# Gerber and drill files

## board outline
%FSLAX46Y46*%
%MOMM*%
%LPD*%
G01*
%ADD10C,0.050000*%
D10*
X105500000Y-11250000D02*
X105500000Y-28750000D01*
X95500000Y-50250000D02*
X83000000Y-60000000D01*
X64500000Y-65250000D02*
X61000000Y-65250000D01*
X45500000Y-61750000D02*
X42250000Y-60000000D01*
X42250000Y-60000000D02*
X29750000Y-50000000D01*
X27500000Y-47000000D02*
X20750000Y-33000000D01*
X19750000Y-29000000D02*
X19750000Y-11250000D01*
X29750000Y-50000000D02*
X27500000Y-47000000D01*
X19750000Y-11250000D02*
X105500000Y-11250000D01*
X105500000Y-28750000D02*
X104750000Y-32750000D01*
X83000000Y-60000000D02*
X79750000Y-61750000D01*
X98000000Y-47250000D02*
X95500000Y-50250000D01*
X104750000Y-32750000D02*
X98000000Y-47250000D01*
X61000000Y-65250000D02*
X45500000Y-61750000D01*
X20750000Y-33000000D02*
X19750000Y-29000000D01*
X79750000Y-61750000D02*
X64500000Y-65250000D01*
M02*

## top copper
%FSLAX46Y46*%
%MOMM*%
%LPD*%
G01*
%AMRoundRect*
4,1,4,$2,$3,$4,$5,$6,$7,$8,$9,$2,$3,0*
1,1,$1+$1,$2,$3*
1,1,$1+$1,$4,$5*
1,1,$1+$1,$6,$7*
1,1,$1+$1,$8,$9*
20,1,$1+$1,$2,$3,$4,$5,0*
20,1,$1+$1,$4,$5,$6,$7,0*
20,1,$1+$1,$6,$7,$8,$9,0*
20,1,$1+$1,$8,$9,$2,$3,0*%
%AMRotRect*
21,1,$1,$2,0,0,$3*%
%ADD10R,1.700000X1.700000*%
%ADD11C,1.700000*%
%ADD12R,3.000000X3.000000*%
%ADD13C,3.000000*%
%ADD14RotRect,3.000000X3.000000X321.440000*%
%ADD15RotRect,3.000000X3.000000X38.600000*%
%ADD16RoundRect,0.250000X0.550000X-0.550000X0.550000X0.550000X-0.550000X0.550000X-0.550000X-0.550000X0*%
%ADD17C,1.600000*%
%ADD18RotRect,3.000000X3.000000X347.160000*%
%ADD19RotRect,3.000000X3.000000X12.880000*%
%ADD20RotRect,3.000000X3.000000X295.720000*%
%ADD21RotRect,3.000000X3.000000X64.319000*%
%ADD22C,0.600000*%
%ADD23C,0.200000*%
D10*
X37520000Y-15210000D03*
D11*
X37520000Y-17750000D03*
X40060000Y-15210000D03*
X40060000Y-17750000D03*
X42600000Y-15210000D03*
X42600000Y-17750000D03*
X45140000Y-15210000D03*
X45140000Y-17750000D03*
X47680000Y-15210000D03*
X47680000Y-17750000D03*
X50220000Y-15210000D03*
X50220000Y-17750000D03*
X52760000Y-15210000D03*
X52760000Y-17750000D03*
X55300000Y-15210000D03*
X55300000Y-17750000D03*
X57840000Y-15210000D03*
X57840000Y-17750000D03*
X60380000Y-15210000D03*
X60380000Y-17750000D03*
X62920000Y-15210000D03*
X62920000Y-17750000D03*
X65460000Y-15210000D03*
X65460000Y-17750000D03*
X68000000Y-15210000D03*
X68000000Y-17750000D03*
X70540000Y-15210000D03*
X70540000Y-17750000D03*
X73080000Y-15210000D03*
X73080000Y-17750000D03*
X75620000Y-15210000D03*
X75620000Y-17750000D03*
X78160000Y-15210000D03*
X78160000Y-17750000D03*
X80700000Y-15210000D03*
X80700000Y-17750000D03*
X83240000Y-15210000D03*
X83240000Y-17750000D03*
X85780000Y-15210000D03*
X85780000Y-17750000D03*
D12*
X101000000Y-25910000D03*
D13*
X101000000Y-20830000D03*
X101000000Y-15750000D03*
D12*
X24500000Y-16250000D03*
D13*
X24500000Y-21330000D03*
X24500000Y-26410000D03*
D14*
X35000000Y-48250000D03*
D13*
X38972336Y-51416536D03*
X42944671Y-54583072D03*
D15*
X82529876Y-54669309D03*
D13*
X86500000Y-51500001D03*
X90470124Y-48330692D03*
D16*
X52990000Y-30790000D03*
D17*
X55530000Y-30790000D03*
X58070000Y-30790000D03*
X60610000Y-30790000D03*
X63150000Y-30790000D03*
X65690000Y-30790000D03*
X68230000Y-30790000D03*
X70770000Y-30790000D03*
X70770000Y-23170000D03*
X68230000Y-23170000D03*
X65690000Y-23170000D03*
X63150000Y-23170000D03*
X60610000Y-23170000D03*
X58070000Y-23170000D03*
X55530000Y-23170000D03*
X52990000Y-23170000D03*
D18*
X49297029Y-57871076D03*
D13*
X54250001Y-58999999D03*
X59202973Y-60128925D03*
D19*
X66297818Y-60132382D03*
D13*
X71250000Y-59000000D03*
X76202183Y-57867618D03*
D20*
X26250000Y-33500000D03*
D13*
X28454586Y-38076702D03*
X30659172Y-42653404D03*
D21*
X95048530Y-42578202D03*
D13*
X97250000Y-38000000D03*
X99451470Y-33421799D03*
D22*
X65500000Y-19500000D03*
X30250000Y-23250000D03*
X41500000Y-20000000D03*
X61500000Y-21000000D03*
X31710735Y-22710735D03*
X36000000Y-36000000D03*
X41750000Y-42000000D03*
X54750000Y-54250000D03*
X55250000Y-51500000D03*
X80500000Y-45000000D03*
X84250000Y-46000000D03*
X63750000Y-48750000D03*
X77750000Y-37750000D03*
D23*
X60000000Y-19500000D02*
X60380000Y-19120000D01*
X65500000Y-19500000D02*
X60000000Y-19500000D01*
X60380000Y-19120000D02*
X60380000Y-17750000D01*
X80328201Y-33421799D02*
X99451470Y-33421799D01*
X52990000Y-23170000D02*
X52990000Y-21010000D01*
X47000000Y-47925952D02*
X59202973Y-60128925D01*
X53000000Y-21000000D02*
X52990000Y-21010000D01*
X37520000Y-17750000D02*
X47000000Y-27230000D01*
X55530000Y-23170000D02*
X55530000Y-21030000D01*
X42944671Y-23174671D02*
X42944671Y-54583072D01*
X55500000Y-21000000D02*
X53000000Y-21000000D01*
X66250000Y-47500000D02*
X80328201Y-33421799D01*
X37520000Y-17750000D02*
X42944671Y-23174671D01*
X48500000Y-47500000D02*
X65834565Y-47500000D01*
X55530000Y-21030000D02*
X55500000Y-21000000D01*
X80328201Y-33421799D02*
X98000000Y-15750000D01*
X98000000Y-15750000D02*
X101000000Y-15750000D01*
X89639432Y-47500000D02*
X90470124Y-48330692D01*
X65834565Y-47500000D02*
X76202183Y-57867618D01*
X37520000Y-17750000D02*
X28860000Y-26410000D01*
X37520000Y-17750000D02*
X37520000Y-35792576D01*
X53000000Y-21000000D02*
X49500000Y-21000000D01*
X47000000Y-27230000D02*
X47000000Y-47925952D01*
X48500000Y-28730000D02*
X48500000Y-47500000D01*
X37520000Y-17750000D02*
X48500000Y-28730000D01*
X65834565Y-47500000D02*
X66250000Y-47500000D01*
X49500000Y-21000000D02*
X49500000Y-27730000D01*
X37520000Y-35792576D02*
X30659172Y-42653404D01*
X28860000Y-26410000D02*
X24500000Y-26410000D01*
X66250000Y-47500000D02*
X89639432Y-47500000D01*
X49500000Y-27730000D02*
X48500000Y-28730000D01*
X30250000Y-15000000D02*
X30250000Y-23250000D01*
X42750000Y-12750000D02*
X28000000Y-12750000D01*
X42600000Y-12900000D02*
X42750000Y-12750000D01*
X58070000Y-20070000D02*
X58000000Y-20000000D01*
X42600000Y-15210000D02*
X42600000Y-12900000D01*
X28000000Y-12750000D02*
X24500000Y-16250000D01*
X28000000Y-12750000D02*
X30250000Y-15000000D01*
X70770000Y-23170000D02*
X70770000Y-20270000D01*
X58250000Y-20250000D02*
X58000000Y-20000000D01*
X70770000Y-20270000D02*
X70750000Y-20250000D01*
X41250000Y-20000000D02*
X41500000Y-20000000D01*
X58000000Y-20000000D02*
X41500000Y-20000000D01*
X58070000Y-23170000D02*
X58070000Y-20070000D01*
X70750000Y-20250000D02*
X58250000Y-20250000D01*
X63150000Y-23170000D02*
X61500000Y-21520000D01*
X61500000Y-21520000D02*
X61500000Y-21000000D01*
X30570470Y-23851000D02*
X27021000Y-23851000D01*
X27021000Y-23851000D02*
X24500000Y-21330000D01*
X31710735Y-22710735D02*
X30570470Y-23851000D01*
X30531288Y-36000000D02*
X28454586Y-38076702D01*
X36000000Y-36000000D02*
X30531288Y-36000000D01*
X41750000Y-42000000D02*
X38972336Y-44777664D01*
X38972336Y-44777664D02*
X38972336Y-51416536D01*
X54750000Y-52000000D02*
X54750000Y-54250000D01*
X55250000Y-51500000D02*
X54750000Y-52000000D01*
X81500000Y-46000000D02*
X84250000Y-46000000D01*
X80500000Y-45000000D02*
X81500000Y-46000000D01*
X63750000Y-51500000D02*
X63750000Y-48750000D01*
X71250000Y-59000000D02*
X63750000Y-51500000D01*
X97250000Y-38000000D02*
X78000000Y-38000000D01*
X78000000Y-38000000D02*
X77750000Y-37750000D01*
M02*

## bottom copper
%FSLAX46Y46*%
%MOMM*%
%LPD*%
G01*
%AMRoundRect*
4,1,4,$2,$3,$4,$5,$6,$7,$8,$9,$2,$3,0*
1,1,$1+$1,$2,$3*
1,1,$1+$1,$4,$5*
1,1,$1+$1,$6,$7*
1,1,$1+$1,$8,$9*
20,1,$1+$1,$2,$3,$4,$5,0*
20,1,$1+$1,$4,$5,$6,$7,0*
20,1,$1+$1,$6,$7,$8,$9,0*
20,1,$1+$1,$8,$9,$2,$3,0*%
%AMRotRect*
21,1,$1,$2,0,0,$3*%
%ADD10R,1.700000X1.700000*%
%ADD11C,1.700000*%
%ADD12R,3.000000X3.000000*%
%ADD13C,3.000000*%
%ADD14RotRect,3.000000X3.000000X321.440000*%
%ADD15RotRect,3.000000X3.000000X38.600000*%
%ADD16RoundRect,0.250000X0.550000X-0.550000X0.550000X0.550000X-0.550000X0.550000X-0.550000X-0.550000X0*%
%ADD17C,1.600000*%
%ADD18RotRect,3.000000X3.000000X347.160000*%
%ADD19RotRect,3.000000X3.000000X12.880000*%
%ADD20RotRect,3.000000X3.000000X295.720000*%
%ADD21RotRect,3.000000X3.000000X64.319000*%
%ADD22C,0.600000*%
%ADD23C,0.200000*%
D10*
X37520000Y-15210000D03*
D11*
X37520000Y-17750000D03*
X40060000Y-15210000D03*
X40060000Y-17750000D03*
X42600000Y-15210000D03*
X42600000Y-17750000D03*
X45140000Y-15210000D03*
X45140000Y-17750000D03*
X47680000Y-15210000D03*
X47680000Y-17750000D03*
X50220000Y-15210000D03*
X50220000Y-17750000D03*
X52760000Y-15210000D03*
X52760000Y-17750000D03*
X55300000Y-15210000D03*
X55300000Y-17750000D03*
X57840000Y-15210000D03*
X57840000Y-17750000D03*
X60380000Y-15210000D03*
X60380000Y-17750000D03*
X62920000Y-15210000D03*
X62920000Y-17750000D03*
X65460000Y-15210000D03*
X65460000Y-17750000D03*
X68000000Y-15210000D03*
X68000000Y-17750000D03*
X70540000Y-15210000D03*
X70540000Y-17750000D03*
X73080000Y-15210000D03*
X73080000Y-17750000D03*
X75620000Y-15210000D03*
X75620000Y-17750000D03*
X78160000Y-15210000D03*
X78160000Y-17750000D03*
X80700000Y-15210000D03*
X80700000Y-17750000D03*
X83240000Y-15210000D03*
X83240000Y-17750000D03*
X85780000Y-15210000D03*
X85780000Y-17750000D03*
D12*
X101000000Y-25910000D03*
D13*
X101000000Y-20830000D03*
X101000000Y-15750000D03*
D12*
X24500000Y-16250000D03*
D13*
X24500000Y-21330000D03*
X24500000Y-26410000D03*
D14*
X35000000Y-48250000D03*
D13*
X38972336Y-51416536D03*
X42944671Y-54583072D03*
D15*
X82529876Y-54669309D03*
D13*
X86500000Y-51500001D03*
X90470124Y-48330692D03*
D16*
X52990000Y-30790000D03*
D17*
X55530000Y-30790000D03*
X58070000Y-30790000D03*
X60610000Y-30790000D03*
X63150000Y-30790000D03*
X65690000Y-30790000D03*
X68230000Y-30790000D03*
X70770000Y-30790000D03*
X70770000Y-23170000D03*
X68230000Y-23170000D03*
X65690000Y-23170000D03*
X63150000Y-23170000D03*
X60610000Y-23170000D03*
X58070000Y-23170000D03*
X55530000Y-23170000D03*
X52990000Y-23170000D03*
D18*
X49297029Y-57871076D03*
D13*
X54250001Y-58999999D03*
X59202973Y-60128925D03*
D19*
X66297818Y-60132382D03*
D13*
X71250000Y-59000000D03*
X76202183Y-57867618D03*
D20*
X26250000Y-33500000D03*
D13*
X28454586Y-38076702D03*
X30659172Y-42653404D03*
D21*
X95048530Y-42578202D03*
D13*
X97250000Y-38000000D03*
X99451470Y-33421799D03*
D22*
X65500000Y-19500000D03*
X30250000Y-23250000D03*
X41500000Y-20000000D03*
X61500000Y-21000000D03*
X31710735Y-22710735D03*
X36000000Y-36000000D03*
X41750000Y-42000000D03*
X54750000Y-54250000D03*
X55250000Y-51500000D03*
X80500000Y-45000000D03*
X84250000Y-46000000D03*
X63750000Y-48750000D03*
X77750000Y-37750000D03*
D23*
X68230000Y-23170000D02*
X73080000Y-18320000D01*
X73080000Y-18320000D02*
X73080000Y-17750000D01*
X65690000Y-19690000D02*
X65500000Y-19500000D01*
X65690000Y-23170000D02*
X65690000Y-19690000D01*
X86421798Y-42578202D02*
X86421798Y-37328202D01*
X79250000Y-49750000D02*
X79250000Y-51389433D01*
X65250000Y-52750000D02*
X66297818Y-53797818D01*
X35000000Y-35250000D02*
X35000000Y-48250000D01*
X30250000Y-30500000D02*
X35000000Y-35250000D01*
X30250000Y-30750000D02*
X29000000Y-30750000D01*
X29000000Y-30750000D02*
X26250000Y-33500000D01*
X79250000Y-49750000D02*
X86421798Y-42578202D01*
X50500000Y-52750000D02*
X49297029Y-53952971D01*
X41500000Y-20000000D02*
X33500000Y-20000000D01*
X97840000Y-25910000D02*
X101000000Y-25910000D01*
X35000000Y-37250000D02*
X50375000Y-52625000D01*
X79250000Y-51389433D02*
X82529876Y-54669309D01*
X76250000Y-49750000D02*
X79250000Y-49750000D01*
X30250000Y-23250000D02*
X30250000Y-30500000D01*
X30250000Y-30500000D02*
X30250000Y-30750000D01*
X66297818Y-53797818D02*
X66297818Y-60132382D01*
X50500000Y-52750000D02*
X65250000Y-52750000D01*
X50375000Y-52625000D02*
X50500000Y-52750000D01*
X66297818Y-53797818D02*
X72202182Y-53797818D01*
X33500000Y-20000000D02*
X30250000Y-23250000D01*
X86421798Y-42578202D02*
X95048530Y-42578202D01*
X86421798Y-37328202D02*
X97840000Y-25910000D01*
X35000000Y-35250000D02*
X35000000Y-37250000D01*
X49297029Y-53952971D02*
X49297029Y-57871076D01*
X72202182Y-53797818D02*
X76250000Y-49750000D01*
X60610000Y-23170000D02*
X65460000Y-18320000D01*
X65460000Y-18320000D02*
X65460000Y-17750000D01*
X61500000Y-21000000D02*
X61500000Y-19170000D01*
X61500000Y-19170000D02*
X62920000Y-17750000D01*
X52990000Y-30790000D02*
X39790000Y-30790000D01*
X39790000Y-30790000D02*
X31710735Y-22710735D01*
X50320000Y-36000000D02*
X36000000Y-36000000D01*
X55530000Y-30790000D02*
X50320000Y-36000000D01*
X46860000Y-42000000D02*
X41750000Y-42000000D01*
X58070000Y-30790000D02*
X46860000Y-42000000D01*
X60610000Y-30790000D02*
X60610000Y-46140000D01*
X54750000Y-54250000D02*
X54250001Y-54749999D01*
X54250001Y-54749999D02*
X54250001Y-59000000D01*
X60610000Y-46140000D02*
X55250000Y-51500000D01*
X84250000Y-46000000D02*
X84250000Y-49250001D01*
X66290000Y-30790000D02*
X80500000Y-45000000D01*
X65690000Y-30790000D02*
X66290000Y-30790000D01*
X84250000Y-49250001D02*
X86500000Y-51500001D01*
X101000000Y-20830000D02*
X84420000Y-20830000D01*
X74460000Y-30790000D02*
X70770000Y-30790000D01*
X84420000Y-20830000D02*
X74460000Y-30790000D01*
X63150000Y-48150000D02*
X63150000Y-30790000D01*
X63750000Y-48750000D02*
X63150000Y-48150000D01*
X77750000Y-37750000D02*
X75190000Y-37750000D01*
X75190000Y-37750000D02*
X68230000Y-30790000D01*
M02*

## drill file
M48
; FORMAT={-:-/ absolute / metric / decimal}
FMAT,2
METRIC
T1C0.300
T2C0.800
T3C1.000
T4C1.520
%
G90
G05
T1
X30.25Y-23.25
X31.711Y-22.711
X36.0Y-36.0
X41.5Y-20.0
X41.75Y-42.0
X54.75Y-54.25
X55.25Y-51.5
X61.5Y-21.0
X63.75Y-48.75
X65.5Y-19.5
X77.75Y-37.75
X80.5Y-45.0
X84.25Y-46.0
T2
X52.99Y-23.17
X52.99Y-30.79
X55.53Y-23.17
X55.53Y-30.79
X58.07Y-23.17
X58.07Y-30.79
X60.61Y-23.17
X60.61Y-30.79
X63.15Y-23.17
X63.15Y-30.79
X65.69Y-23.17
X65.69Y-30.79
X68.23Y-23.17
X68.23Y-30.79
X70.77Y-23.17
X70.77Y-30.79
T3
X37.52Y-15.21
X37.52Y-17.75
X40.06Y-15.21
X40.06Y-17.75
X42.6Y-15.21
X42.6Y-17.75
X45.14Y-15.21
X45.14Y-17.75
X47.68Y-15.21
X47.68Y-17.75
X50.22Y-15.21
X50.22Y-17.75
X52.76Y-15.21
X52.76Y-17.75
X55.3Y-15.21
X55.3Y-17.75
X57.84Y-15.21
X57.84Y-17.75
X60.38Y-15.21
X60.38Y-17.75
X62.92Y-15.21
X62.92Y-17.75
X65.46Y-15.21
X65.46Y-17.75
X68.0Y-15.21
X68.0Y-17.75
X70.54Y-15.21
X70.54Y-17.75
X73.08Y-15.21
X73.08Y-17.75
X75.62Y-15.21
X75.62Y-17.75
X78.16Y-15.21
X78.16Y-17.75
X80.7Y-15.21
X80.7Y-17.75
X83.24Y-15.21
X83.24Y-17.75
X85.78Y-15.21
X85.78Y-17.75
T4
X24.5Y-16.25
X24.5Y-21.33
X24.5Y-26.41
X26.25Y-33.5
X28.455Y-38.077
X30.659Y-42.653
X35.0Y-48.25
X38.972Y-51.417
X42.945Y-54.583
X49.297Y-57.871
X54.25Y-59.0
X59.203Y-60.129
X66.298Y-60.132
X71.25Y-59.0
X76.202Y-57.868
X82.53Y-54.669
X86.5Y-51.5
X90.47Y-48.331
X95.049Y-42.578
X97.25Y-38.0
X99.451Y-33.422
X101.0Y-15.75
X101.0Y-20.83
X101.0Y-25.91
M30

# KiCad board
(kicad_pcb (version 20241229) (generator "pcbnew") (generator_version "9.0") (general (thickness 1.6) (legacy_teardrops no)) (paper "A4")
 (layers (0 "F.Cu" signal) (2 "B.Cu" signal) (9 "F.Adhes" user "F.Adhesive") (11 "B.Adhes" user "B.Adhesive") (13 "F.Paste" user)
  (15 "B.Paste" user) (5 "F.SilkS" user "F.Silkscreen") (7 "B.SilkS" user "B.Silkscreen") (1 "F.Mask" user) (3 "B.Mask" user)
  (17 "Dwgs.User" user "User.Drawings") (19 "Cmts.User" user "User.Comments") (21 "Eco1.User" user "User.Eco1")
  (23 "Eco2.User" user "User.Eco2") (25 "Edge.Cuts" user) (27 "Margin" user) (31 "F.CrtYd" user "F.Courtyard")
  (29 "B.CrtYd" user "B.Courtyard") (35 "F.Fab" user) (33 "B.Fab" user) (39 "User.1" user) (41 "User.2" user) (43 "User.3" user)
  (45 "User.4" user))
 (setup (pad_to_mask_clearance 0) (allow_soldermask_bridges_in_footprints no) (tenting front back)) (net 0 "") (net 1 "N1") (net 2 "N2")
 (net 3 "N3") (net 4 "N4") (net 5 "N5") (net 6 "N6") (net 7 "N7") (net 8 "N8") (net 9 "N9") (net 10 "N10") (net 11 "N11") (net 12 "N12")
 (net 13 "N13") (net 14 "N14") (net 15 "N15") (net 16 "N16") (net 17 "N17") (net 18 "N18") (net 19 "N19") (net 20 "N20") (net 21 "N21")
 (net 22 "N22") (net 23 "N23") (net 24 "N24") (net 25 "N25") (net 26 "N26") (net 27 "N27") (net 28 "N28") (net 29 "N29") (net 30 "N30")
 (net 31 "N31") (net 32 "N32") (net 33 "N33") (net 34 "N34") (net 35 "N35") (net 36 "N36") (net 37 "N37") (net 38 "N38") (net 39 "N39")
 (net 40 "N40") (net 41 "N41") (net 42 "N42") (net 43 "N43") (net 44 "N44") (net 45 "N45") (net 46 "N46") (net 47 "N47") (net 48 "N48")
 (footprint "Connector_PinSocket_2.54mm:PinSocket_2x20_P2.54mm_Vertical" (layer "F.Cu") (at 37.52 15.21 90)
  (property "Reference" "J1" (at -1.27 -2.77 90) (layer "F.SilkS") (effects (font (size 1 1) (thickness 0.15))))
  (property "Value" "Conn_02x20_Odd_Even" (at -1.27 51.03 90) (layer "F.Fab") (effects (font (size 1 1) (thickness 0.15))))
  (pad "1" thru_hole rect (at 0 0 90) (size 1.7 1.7) (drill 1) (layers "*.Cu" "*.Mask") (remove_unused_layers no) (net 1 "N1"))
  (pad "2" thru_hole circle (at -2.54 0 90) (size 1.7 1.7) (drill 1) (layers "*.Cu" "*.Mask") (remove_unused_layers no) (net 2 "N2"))
  (pad "3" thru_hole circle (at 0 2.54 90) (size 1.7 1.7) (drill 1) (layers "*.Cu" "*.Mask") (remove_unused_layers no) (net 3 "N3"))
  (pad "4" thru_hole circle (at -2.54 2.54 90) (size 1.7 1.7) (drill 1) (layers "*.Cu" "*.Mask") (remove_unused_layers no) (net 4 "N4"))
  (pad "5" thru_hole circle (at 0 5.08 90) (size 1.7 1.7) (drill 1) (layers "*.Cu" "*.Mask") (remove_unused_layers no) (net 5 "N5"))
  (pad "6" thru_hole circle (at -2.54 5.08 90) (size 1.7 1.7) (drill 1) (layers "*.Cu" "*.Mask") (remove_unused_layers no) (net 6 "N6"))
  (pad "7" thru_hole circle (at 0 7.62 90) (size 1.7 1.7) (drill 1) (layers "*.Cu" "*.Mask") (remove_unused_layers no) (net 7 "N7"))
  (pad "8" thru_hole circle (at -2.54 7.62 90) (size 1.7 1.7) (drill 1) (layers "*.Cu" "*.Mask") (remove_unused_layers no) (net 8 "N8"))
  (pad "9" thru_hole circle (at 0 10.16 90) (size 1.7 1.7) (drill 1) (layers "*.Cu" "*.Mask") (remove_unused_layers no) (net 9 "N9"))
  (pad "10" thru_hole circle (at -2.54 10.16 90) (size 1.7 1.7) (drill 1) (layers "*.Cu" "*.Mask") (remove_unused_layers no) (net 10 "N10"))
  (pad "11" thru_hole circle (at 0 12.7 90) (size 1.7 1.7) (drill 1) (layers "*.Cu" "*.Mask") (remove_unused_layers no) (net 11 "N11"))
  (pad "12" thru_hole circle (at -2.54 12.7 90) (size 1.7 1.7) (drill 1) (layers "*.Cu" "*.Mask") (remove_unused_layers no) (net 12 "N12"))
  (pad "13" thru_hole circle (at 0 15.24 90) (size 1.7 1.7) (drill 1) (layers "*.Cu" "*.Mask") (remove_unused_layers no) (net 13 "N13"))
  (pad "14" thru_hole circle (at -2.54 15.24 90) (size 1.7 1.7) (drill 1) (layers "*.Cu" "*.Mask") (remove_unused_layers no) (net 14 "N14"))
  (pad "15" thru_hole circle (at 0 17.78 90) (size 1.7 1.7) (drill 1) (layers "*.Cu" "*.Mask") (remove_unused_layers no) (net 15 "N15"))
  (pad "16" thru_hole circle (at -2.54 17.78 90) (size 1.7 1.7) (drill 1) (layers "*.Cu" "*.Mask") (remove_unused_layers no) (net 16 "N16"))
  (pad "17" thru_hole circle (at 0 20.32 90) (size 1.7 1.7) (drill 1) (layers "*.Cu" "*.Mask") (remove_unused_layers no) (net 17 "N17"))
  (pad "18" thru_hole circle (at -2.54 20.32 90) (size 1.7 1.7) (drill 1) (layers "*.Cu" "*.Mask") (remove_unused_layers no) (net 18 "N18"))
  (pad "19" thru_hole circle (at 0 22.86 90) (size 1.7 1.7) (drill 1) (layers "*.Cu" "*.Mask") (remove_unused_layers no) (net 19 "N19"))
  (pad "20" thru_hole circle (at -2.54 22.86 90) (size 1.7 1.7) (drill 1) (layers "*.Cu" "*.Mask") (remove_unused_layers no) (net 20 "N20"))
  (pad "21" thru_hole circle (at 0 25.4 90) (size 1.7 1.7) (drill 1) (layers "*.Cu" "*.Mask") (remove_unused_layers no) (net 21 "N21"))
  (pad "22" thru_hole circle (at -2.54 25.4 90) (size 1.7 1.7) (drill 1) (layers "*.Cu" "*.Mask") (remove_unused_layers no) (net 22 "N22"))
  (pad "23" thru_hole circle (at 0 27.94 90) (size 1.7 1.7) (drill 1) (layers "*.Cu" "*.Mask") (remove_unused_layers no) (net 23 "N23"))
  (pad "24" thru_hole circle (at -2.54 27.94 90) (size 1.7 1.7) (drill 1) (layers "*.Cu" "*.Mask") (remove_unused_layers no) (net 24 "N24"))
  (pad "25" thru_hole circle (at 0 30.48 90) (size 1.7 1.7) (drill 1) (layers "*.Cu" "*.Mask") (remove_unused_layers no) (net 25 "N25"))
  (pad "26" thru_hole circle (at -2.54 30.48 90) (size 1.7 1.7) (drill 1) (layers "*.Cu" "*.Mask") (remove_unused_layers no) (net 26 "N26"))
  (pad "27" thru_hole circle (at 0 33.02 90) (size 1.7 1.7) (drill 1) (layers "*.Cu" "*.Mask") (remove_unused_layers no) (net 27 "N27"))
  (pad "28" thru_hole circle (at -2.54 33.02 90) (size 1.7 1.7) (drill 1) (layers "*.Cu" "*.Mask") (remove_unused_layers no) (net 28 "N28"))
  (pad "29" thru_hole circle (at 0 35.56 90) (size 1.7 1.7) (drill 1) (layers "*.Cu" "*.Mask") (remove_unused_layers no) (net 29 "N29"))
  (pad "30" thru_hole circle (at -2.54 35.56 90) (size 1.7 1.7) (drill 1) (layers "*.Cu" "*.Mask") (remove_unused_layers no) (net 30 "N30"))
  (pad "31" thru_hole circle (at 0 38.1 90) (size 1.7 1.7) (drill 1) (layers "*.Cu" "*.Mask") (remove_unused_layers no) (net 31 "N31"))
  (pad "32" thru_hole circle (at -2.54 38.1 90) (size 1.7 1.7) (drill 1) (layers "*.Cu" "*.Mask") (remove_unused_layers no) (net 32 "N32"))
  (pad "33" thru_hole circle (at 0 40.64 90) (size 1.7 1.7) (drill 1) (layers "*.Cu" "*.Mask") (remove_unused_layers no) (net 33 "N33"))
  (pad "34" thru_hole circle (at -2.54 40.64 90) (size 1.7 1.7) (drill 1) (layers "*.Cu" "*.Mask") (remove_unused_layers no) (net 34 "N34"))
  (pad "35" thru_hole circle (at 0 43.18 90) (size 1.7 1.7) (drill 1) (layers "*.Cu" "*.Mask") (remove_unused_layers no) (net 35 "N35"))
  (pad "36" thru_hole circle (at -2.54 43.18 90) (size 1.7 1.7) (drill 1) (layers "*.Cu" "*.Mask") (remove_unused_layers no) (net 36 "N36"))
  (pad "37" thru_hole circle (at 0 45.72 90) (size 1.7 1.7) (drill 1) (layers "*.Cu" "*.Mask") (remove_unused_layers no) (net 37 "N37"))
  (pad "38" thru_hole circle (at -2.54 45.72 90) (size 1.7 1.7) (drill 1) (layers "*.Cu" "*.Mask") (remove_unused_layers no) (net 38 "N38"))
  (pad "39" thru_hole circle (at 0 48.26 90) (size 1.7 1.7) (drill 1) (layers "*.Cu" "*.Mask") (remove_unused_layers no) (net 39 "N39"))
  (pad "40" thru_hole circle (at -2.54 48.26 90) (size 1.7 1.7) (drill 1) (layers "*.Cu" "*.Mask") (remove_unused_layers no) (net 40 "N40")))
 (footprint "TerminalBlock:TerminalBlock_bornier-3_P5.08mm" (layer "F.Cu") (at 101 25.91 90)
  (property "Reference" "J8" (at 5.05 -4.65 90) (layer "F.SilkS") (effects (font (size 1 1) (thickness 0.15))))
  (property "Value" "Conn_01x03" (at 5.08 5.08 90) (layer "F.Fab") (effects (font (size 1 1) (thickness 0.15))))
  (pad "1" thru_hole rect (at 0 0 90) (size 3 3) (drill 1.52) (layers "*.Cu" "*.Mask") (remove_unused_layers no) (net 5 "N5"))
  (pad "2" thru_hole circle (at 5.08 0 90) (size 3 3) (drill 1.52) (layers "*.Cu" "*.Mask") (remove_unused_layers no) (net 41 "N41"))
  (pad "3" thru_hole circle (at 10.16 0 90) (size 3 3) (drill 1.52) (layers "*.Cu" "*.Mask") (remove_unused_layers no) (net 2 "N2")))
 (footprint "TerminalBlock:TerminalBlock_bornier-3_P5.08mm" (layer "F.Cu") (at 24.5 16.25 -90)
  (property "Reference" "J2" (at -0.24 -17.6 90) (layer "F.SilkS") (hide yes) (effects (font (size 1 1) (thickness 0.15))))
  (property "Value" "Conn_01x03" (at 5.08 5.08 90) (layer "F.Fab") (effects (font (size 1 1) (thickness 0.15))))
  (pad "1" thru_hole rect (at 0 0 270) (size 3 3) (drill 1.52) (layers "*.Cu" "*.Mask") (remove_unused_layers no) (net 5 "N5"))
  (pad "2" thru_hole circle (at 5.08 0 270) (size 3 3) (drill 1.52) (layers "*.Cu" "*.Mask") (remove_unused_layers no) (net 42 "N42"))
  (pad "3" thru_hole circle (at 10.16 0 270) (size 3 3) (drill 1.52) (layers "*.Cu" "*.Mask") (remove_unused_layers no) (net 2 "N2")))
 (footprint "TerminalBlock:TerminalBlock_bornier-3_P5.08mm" (layer "F.Cu") (at 35 48.25 -38.56)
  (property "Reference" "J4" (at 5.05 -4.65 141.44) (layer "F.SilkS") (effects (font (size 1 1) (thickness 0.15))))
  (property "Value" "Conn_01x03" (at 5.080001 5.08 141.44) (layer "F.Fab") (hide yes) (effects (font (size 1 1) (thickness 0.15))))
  (pad "1" thru_hole rect (at 0 0 321.44) (size 3 3) (drill 1.52) (layers "*.Cu" "*.Mask") (remove_unused_layers no) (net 5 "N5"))
  (pad "2" thru_hole circle (at 5.08 0 321.44) (size 3 3) (drill 1.52) (layers "*.Cu" "*.Mask") (remove_unused_layers no) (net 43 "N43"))
  (pad "3" thru_hole circle (at 10.16 0 321.44) (size 3 3) (drill 1.52) (layers "*.Cu" "*.Mask") (remove_unused_layers no) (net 2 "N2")))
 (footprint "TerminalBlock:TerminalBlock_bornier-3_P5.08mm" (layer "F.Cu") (at 82.529876 54.669309 38.6)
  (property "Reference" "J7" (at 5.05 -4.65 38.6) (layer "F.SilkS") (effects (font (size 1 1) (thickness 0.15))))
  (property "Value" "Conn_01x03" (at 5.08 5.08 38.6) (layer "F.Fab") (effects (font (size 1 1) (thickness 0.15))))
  (pad "1" thru_hole rect (at 0 0 38.6) (size 3 3) (drill 1.52) (layers "*.Cu" "*.Mask") (remove_unused_layers no) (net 5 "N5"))
  (pad "2" thru_hole circle (at 5.08 0 38.6) (size 3 3) (drill 1.52) (layers "*.Cu" "*.Mask") (remove_unused_layers no) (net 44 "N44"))
  (pad "3" thru_hole circle (at 10.16 0 38.6) (size 3 3) (drill 1.52) (layers "*.Cu" "*.Mask") (remove_unused_layers no) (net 2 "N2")))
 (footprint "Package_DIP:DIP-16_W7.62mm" (layer "F.Cu") (at 52.99 30.79 90)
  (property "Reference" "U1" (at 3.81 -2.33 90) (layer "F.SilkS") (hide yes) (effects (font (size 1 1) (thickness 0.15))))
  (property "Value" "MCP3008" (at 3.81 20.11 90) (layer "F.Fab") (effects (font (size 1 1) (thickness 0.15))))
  (pad "1" thru_hole roundrect (at 0 0 90) (size 1.6 1.6) (drill 0.8) (layers "*.Cu" "*.Mask") (remove_unused_layers no)
   (roundrect_rratio 0.15625) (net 42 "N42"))
  (pad "2" thru_hole circle (at 0 2.54 90) (size 1.6 1.6) (drill 0.8) (layers "*.Cu" "*.Mask") (remove_unused_layers no) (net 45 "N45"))
  (pad "3" thru_hole circle (at 0 5.08 90) (size 1.6 1.6) (drill 0.8) (layers "*.Cu" "*.Mask") (remove_unused_layers no) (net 43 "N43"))
  (pad "4" thru_hole circle (at 0 7.62 90) (size 1.6 1.6) (drill 0.8) (layers "*.Cu" "*.Mask") (remove_unused_layers no) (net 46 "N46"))
  (pad "5" thru_hole circle (at 0 10.16 90) (size 1.6 1.6) (drill 0.8) (layers "*.Cu" "*.Mask") (remove_unused_layers no) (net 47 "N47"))
  (pad "6" thru_hole circle (at 0 12.7 90) (size 1.6 1.6) (drill 0.8) (layers "*.Cu" "*.Mask") (remove_unused_layers no) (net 44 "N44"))
  (pad "7" thru_hole circle (at 0 15.24 90) (size 1.6 1.6) (drill 0.8) (layers "*.Cu" "*.Mask") (remove_unused_layers no) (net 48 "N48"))
  (pad "8" thru_hole circle (at 0 17.78 90) (size 1.6 1.6) (drill 0.8) (layers "*.Cu" "*.Mask") (remove_unused_layers no) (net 41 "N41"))
  (pad "9" thru_hole circle (at 7.62 17.78 90) (size 1.6 1.6) (drill 0.8) (layers "*.Cu" "*.Mask") (remove_unused_layers no) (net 5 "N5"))
  (pad "10" thru_hole circle (at 7.62 15.24 90) (size 1.6 1.6) (drill 0.8) (layers "*.Cu" "*.Mask") (remove_unused_layers no) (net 30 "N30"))
  (pad "11" thru_hole circle (at 7.62 12.7 90) (size 1.6 1.6) (drill 0.8) (layers "*.Cu" "*.Mask") (remove_unused_layers no) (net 20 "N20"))
  (pad "12" thru_hole circle (at 7.62 10.16 90) (size 1.6 1.6) (drill 0.8) (layers "*.Cu" "*.Mask") (remove_unused_layers no) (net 22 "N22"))
  (pad "13" thru_hole circle (at 7.62 7.62 90) (size 1.6 1.6) (drill 0.8) (layers "*.Cu" "*.Mask") (remove_unused_layers no) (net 24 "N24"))
  (pad "14" thru_hole circle (at 7.62 5.08 90) (size 1.6 1.6) (drill 0.8) (layers "*.Cu" "*.Mask") (remove_unused_layers no) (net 5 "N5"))
  (pad "15" thru_hole circle (at 7.62 2.54 90) (size 1.6 1.6) (drill 0.8) (layers "*.Cu" "*.Mask") (remove_unused_layers no) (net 2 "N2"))
  (pad "16" thru_hole circle (at 7.62 0 90) (size 1.6 1.6) (drill 0.8) (layers "*.Cu" "*.Mask") (remove_unused_layers no) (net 2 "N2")))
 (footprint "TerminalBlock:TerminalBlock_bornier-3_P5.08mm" (layer "F.Cu") (at 49.297029 57.871076 -12.84)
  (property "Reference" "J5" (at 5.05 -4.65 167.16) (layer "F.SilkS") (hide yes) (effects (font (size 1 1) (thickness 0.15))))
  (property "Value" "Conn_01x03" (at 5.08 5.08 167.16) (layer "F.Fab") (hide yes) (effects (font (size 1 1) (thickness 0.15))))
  (pad "1" thru_hole rect (at 0 0 347.16) (size 3 3) (drill 1.52) (layers "*.Cu" "*.Mask") (remove_unused_layers no) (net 5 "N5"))
  (pad "2" thru_hole circle (at 5.08 -0.000001 347.16) (size 3 3) (drill 1.52) (layers "*.Cu" "*.Mask") (remove_unused_layers no)
   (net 46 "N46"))
  (pad "3" thru_hole circle (at 10.16 0 347.16) (size 3 3) (drill 1.52) (layers "*.Cu" "*.Mask") (remove_unused_layers no) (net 2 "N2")))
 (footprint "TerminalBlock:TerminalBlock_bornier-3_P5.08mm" (layer "F.Cu") (at 66.297818 60.132382 12.88)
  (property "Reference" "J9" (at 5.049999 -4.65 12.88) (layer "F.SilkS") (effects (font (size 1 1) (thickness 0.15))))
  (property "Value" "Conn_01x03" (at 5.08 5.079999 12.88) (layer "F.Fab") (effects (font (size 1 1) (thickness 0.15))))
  (pad "1" thru_hole rect (at 0 0 12.88) (size 3 3) (drill 1.52) (layers "*.Cu" "*.Mask") (remove_unused_layers no) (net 5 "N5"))
  (pad "2" thru_hole circle (at 5.08 0 12.88) (size 3 3) (drill 1.52) (layers "*.Cu" "*.Mask") (remove_unused_layers no) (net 47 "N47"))
  (pad "3" thru_hole circle (at 10.16 0 12.88) (size 3 3) (drill 1.52) (layers "*.Cu" "*.Mask") (remove_unused_layers no) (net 2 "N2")))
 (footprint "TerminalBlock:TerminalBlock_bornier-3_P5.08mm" (layer "F.Cu") (at 26.25 33.5 -64.28)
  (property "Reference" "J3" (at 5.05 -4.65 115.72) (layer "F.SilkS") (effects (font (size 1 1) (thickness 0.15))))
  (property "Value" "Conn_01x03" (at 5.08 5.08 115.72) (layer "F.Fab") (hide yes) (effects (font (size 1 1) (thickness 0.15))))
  (pad "1" thru_hole rect (at 0 0 295.72) (size 3 3) (drill 1.52) (layers "*.Cu" "*.Mask") (remove_unused_layers no) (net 5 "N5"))
  (pad "2" thru_hole circle (at 5.08 0 295.72) (size 3 3) (drill 1.52) (layers "*.Cu" "*.Mask") (remove_unused_layers no) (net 45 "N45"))
  (pad "3" thru_hole circle (at 10.16 0 295.72) (size 3 3) (drill 1.52) (layers "*.Cu" "*.Mask") (remove_unused_layers no) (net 2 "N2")))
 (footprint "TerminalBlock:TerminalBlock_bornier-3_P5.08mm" (layer "F.Cu") (at 95.04853 42.578202 64.319)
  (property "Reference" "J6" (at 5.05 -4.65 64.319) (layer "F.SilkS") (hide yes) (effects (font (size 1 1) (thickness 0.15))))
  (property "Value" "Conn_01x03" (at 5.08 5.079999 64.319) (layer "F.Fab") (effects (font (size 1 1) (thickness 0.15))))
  (pad "1" thru_hole rect (at 0 0 64.319) (size 3 3) (drill 1.52) (layers "*.Cu" "*.Mask") (remove_unused_layers no) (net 5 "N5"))
  (pad "2" thru_hole circle (at 5.08 0 64.319) (size 3 3) (drill 1.52) (layers "*.Cu" "*.Mask") (remove_unused_layers no) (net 48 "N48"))
  (pad "3" thru_hole circle (at 10.16 0 64.319) (size 3 3) (drill 1.52) (layers "*.Cu" "*.Mask") (remove_unused_layers no) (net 2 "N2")))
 (gr_line (start 105.5 11.25) (end 105.5 28.75) (stroke (width 0.05) (type default)) (layer "Edge.Cuts"))
 (gr_line (start 95.5 50.25) (end 83 60) (stroke (width 0.05) (type default)) (layer "Edge.Cuts"))
 (gr_line (start 64.5 65.25) (end 61 65.25) (stroke (width 0.05) (type default)) (layer "Edge.Cuts"))
 (gr_line (start 45.5 61.75) (end 42.25 60) (stroke (width 0.05) (type default)) (layer "Edge.Cuts"))
 (gr_line (start 42.25 60) (end 29.75 50) (stroke (width 0.05) (type default)) (layer "Edge.Cuts"))
 (gr_line (start 27.5 47) (end 20.75 33) (stroke (width 0.05) (type default)) (layer "Edge.Cuts"))
 (gr_line (start 19.75 29) (end 19.75 11.25) (stroke (width 0.05) (type default)) (layer "Edge.Cuts"))
 (gr_line (start 29.75 50) (end 27.5 47) (stroke (width 0.05) (type default)) (layer "Edge.Cuts"))
 (gr_line (start 19.75 11.25) (end 105.5 11.25) (stroke (width 0.05) (type default)) (layer "Edge.Cuts"))
 (gr_line (start 105.5 28.75) (end 104.75 32.75) (stroke (width 0.05) (type default)) (layer "Edge.Cuts"))
 (gr_line (start 83 60) (end 79.75 61.75) (stroke (width 0.05) (type default)) (layer "Edge.Cuts"))
 (gr_line (start 98 47.25) (end 95.5 50.25) (stroke (width 0.05) (type default)) (layer "Edge.Cuts"))
 (gr_line (start 104.75 32.75) (end 98 47.25) (stroke (width 0.05) (type default)) (layer "Edge.Cuts"))
 (gr_line (start 61 65.25) (end 45.5 61.75) (stroke (width 0.05) (type default)) (layer "Edge.Cuts"))
 (gr_line (start 20.75 33) (end 19.75 29) (stroke (width 0.05) (type default)) (layer "Edge.Cuts"))
 (gr_line (start 79.75 61.75) (end 64.5 65.25) (stroke (width 0.05) (type default)) (layer "Edge.Cuts"))
 (segment (start 68.23 23.17) (end 73.08 18.32) (width 0.2) (layer "B.Cu") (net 30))
 (segment (start 73.08 18.32) (end 73.08 17.75) (width 0.2) (layer "B.Cu") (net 30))
 (segment (start 60 19.5) (end 60.38 19.12) (width 0.2) (layer "F.Cu") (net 20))
 (segment (start 65.5 19.5) (end 60 19.5) (width 0.2) (layer "F.Cu") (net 20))
 (segment (start 60.38 19.12) (end 60.38 17.75) (width 0.2) (layer "F.Cu") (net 20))
 (via (at 65.5 19.5) (size 0.6) (drill 0.3) (layers "F.Cu" "B.Cu") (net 20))
 (segment (start 65.69 19.69) (end 65.5 19.5) (width 0.2) (layer "B.Cu") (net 20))
 (segment (start 65.69 23.17) (end 65.69 19.69) (width 0.2) (layer "B.Cu") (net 20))
 (segment (start 80.328201 33.421799) (end 99.45147 33.421799) (width 0.2) (layer "F.Cu") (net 2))
 (segment (start 52.99 23.17) (end 52.99 21.01) (width 0.2) (layer "F.Cu") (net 2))
 (segment (start 47 47.925952) (end 59.202973 60.128925) (width 0.2) (layer "F.Cu") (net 2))
 (segment (start 53 21) (end 52.99 21.01) (width 0.2) (layer "F.Cu") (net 2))
 (segment (start 37.52 17.75) (end 47 27.23) (width 0.2) (layer "F.Cu") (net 2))
 (segment (start 55.53 23.17) (end 55.53 21.03) (width 0.2) (layer "F.Cu") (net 2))
 (segment (start 42.944671 23.174671) (end 42.944671 54.583072) (width 0.2) (layer "F.Cu") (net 2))
 (segment (start 55.5 21) (end 53 21) (width 0.2) (layer "F.Cu") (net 2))
 (segment (start 66.25 47.5) (end 80.328201 33.421799) (width 0.2) (layer "F.Cu") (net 2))
 (segment (start 37.52 17.75) (end 42.944671 23.174671) (width 0.2) (layer "F.Cu") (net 2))
 (segment (start 48.5 47.5) (end 65.834565 47.5) (width 0.2) (layer "F.Cu") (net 2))
 (segment (start 55.53 21.03) (end 55.5 21) (width 0.2) (layer "F.Cu") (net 2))
 (segment (start 80.328201 33.421799) (end 98 15.75) (width 0.2) (layer "F.Cu") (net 2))
 (segment (start 98 15.75) (end 101 15.75) (width 0.2) (layer "F.Cu") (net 2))
 (segment (start 89.639432 47.5) (end 90.470124 48.330692) (width 0.2) (layer "F.Cu") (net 2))
 (segment (start 65.834565 47.5) (end 76.202183 57.867618) (width 0.2) (layer "F.Cu") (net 2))
 (segment (start 37.52 17.75) (end 28.86 26.41) (width 0.2) (layer "F.Cu") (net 2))
 (segment (start 37.52 17.75) (end 37.52 35.792576) (width 0.2) (layer "F.Cu") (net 2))
 (segment (start 53 21) (end 49.5 21) (width 0.2) (layer "F.Cu") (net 2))
 (segment (start 47 27.23) (end 47 47.925952) (width 0.2) (layer "F.Cu") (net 2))
 (segment (start 48.5 28.73) (end 48.5 47.5) (width 0.2) (layer "F.Cu") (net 2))
 (segment (start 37.52 17.75) (end 48.5 28.73) (width 0.2) (layer "F.Cu") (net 2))
 (segment (start 65.834565 47.5) (end 66.25 47.5) (width 0.2) (layer "F.Cu") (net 2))
 (segment (start 49.5 21) (end 49.5 27.73) (width 0.2) (layer "F.Cu") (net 2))
 (segment (start 37.52 35.792576) (end 30.659172 42.653404) (width 0.2) (layer "F.Cu") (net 2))
 (segment (start 28.86 26.41) (end 24.5 26.41) (width 0.2) (layer "F.Cu") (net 2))
 (segment (start 66.25 47.5) (end 89.639432 47.5) (width 0.2) (layer "F.Cu") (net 2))
 (segment (start 49.5 27.73) (end 48.5 28.73) (width 0.2) (layer "F.Cu") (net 2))
 (segment (start 30.25 15) (end 30.25 23.25) (width 0.2) (layer "F.Cu") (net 5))
 (segment (start 42.75 12.75) (end 28 12.75) (width 0.2) (layer "F.Cu") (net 5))
 (segment (start 42.6 12.9) (end 42.75 12.75) (width 0.2) (layer "F.Cu") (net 5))
 (segment (start 58.07 20.07) (end 58 20) (width 0.2) (layer "F.Cu") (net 5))
 (segment (start 42.6 15.21) (end 42.6 12.9) (width 0.2) (layer "F.Cu") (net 5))
 (segment (start 28 12.75) (end 24.5 16.25) (width 0.2) (layer "F.Cu") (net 5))
 (segment (start 28 12.75) (end 30.25 15) (width 0.2) (layer "F.Cu") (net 5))
 (segment (start 70.77 23.17) (end 70.77 20.27) (width 0.2) (layer "F.Cu") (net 5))
 (segment (start 58.25 20.25) (end 58 20) (width 0.2) (layer "F.Cu") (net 5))
 (segment (start 70.77 20.27) (end 70.75 20.25) (width 0.2) (layer "F.Cu") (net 5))
 (segment (start 41.25 20) (end 41.5 20) (width 0.2) (layer "F.Cu") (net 5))
 (segment (start 58 20) (end 41.5 20) (width 0.2) (layer "F.Cu") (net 5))
 (segment (start 58.07 23.17) (end 58.07 20.07) (width 0.2) (layer "F.Cu") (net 5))
 (segment (start 70.75 20.25) (end 58.25 20.25) (width 0.2) (layer "F.Cu") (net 5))
 (via (at 30.25 23.25) (size 0.6) (drill 0.3) (layers "F.Cu" "B.Cu") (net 5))
 (via (at 41.5 20) (size 0.6) (drill 0.3) (layers "F.Cu" "B.Cu") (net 5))
 (segment (start 86.421798 42.578202) (end 86.421798 37.328202) (width 0.2) (layer "B.Cu") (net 5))
 (segment (start 79.25 49.75) (end 79.25 51.389433) (width 0.2) (layer "B.Cu") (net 5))
 (segment (start 65.25 52.75) (end 66.297818 53.797818) (width 0.2) (layer "B.Cu") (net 5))
 (segment (start 35 35.25) (end 35 48.25) (width 0.2) (layer "B.Cu") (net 5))
 (segment (start 30.25 30.5) (end 35 35.25) (width 0.2) (layer "B.Cu") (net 5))
 (segment (start 30.25 30.75) (end 29 30.75) (width 0.2) (layer "B.Cu") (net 5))
 (segment (start 29 30.75) (end 26.25 33.5) (width 0.2) (layer "B.Cu") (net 5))
 (segment (start 79.25 49.75) (end 86.421798 42.578202) (width 0.2) (layer "B.Cu") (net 5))
 (segment (start 50.5 52.75) (end 49.297029 53.952971) (width 0.2) (layer "B.Cu") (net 5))
 (segment (start 41.5 20) (end 33.5 20) (width 0.2) (layer "B.Cu") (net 5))
 (segment (start 97.84 25.91) (end 101 25.91) (width 0.2) (layer "B.Cu") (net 5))
 (segment (start 35 37.25) (end 50.375 52.625) (width 0.2) (layer "B.Cu") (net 5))
 (segment (start 79.25 51.389433) (end 82.529876 54.669309) (width 0.2) (layer "B.Cu") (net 5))
 (segment (start 76.25 49.75) (end 79.25 49.75) (width 0.2) (layer "B.Cu") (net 5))
 (segment (start 30.25 23.25) (end 30.25 30.5) (width 0.2) (layer "B.Cu") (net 5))
 (segment (start 30.25 30.5) (end 30.25 30.75) (width 0.2) (layer "B.Cu") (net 5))
 (segment (start 66.297818 53.797818) (end 66.297818 60.132382) (width 0.2) (layer "B.Cu") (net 5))
 (segment (start 50.5 52.75) (end 65.25 52.75) (width 0.2) (layer "B.Cu") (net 5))
 (segment (start 50.375 52.625) (end 50.5 52.75) (width 0.2) (layer "B.Cu") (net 5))
 (segment (start 66.297818 53.797818) (end 72.202182 53.797818) (width 0.2) (layer "B.Cu") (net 5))
 (segment (start 33.5 20) (end 30.25 23.25) (width 0.2) (layer "B.Cu") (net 5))
 (segment (start 86.421798 42.578202) (end 95.04853 42.578202) (width 0.2) (layer "B.Cu") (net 5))
 (segment (start 86.421798 37.328202) (end 97.84 25.91) (width 0.2) (layer "B.Cu") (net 5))
 (segment (start 35 35.25) (end 35 37.25) (width 0.2) (layer "B.Cu") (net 5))
 (segment (start 49.297029 53.952971) (end 49.297029 57.871076) (width 0.2) (layer "B.Cu") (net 5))
 (segment (start 72.202182 53.797818) (end 76.25 49.75) (width 0.2) (layer "B.Cu") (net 5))
 (segment (start 60.61 23.17) (end 65.46 18.32) (width 0.2) (layer "B.Cu") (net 24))
 (segment (start 65.46 18.32) (end 65.46 17.75) (width 0.2) (layer "B.Cu") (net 24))
 (segment (start 63.15 23.17) (end 61.5 21.52) (width 0.2) (layer "F.Cu") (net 22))
 (segment (start 61.5 21.52) (end 61.5 21) (width 0.2) (layer "F.Cu") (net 22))
 (via (at 61.5 21) (size 0.6) (drill 0.3) (layers "F.Cu" "B.Cu") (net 22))
 (segment (start 61.5 21) (end 61.5 19.17) (width 0.2) (layer "B.Cu") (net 22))
 (segment (start 61.5 19.17) (end 62.92 17.75) (width 0.2) (layer "B.Cu") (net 22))
 (segment (start 30.57047 23.851) (end 27.021 23.851) (width 0.2) (layer "F.Cu") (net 42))
 (segment (start 27.021 23.851) (end 24.5 21.33) (width 0.2) (layer "F.Cu") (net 42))
 (segment (start 31.710735 22.710735) (end 30.57047 23.851) (width 0.2) (layer "F.Cu") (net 42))
 (via (at 31.710735 22.710735) (size 0.6) (drill 0.3) (layers "F.Cu" "B.Cu") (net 42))
 (segment (start 52.99 30.79) (end 39.79 30.79) (width 0.2) (layer "B.Cu") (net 42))
 (segment (start 39.79 30.79) (end 31.710735 22.710735) (width 0.2) (layer "B.Cu") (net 42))
 (segment (start 30.531288 36) (end 28.454586 38.076702) (width 0.2) (layer "F.Cu") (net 45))
 (segment (start 36 36) (end 30.531288 36) (width 0.2) (layer "F.Cu") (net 45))
 (via (at 36 36) (size 0.6) (drill 0.3) (layers "F.Cu" "B.Cu") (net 45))
 (segment (start 50.32 36) (end 36 36) (width 0.2) (layer "B.Cu") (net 45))
 (segment (start 55.53 30.79) (end 50.32 36) (width 0.2) (layer "B.Cu") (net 45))
 (segment (start 41.75 42) (end 38.972336 44.777664) (width 0.2) (layer "F.Cu") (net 43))
 (segment (start 38.972336 44.777664) (end 38.972336 51.416536) (width 0.2) (layer "F.Cu") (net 43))
 (via (at 41.75 42) (size 0.6) (drill 0.3) (layers "F.Cu" "B.Cu") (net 43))
 (segment (start 46.86 42) (end 41.75 42) (width 0.2) (layer "B.Cu") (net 43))
 (segment (start 58.07 30.79) (end 46.86 42) (width 0.2) (layer "B.Cu") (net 43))
 (segment (start 54.75 52) (end 54.75 54.25) (width 0.2) (layer "F.Cu") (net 46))
 (segment (start 55.25 51.5) (end 54.75 52) (width 0.2) (layer "F.Cu") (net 46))
 (via (at 54.75 54.25) (size 0.6) (drill 0.3) (layers "F.Cu" "B.Cu") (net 46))
 (via (at 55.25 51.5) (size 0.6) (drill 0.3) (layers "F.Cu" "B.Cu") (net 46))
 (segment (start 60.61 30.79) (end 60.61 46.14) (width 0.2) (layer "B.Cu") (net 46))
 (segment (start 54.75 54.25) (end 54.250001 54.749999) (width 0.2) (layer "B.Cu") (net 46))
 (segment (start 54.250001 54.749999) (end 54.250001 59) (width 0.2) (layer "B.Cu") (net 46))
 (segment (start 60.61 46.14) (end 55.25 51.5) (width 0.2) (layer "B.Cu") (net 46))
 (segment (start 81.5 46) (end 84.25 46) (width 0.2) (layer "F.Cu") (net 44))
 (segment (start 80.5 45) (end 81.5 46) (width 0.2) (layer "F.Cu") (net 44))
 (via (at 80.5 45) (size 0.6) (drill 0.3) (layers "F.Cu" "B.Cu") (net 44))
 (via (at 84.25 46) (size 0.6) (drill 0.3) (layers "F.Cu" "B.Cu") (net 44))
 (segment (start 84.25 46) (end 84.25 49.250001) (width 0.2) (layer "B.Cu") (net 44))
 (segment (start 66.29 30.79) (end 80.5 45) (width 0.2) (layer "B.Cu") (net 44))
 (segment (start 65.69 30.79) (end 66.29 30.79) (width 0.2) (layer "B.Cu") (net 44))
 (segment (start 84.25 49.250001) (end 86.5 51.500001) (width 0.2) (layer "B.Cu") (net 44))
 (segment (start 101 20.83) (end 84.42 20.83) (width 0.2) (layer "B.Cu") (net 41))
 (segment (start 74.46 30.79) (end 70.77 30.79) (width 0.2) (layer "B.Cu") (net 41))
 (segment (start 84.42 20.83) (end 74.46 30.79) (width 0.2) (layer "B.Cu") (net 41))
 (segment (start 63.75 51.5) (end 63.75 48.75) (width 0.2) (layer "F.Cu") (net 47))
 (segment (start 71.25 59) (end 63.75 51.5) (width 0.2) (layer "F.Cu") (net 47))
 (via (at 63.75 48.75) (size 0.6) (drill 0.3) (layers "F.Cu" "B.Cu") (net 47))
 (segment (start 63.15 48.15) (end 63.15 30.79) (width 0.2) (layer "B.Cu") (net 47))
 (segment (start 63.75 48.75) (end 63.15 48.15) (width 0.2) (layer "B.Cu") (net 47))
 (segment (start 97.25 38) (end 78 38) (width 0.2) (layer "F.Cu") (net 48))
 (segment (start 78 38) (end 77.75 37.75) (width 0.2) (layer "F.Cu") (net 48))
 (via (at 77.75 37.75) (size 0.6) (drill 0.3) (layers "F.Cu" "B.Cu") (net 48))
 (segment (start 77.75 37.75) (end 75.19 37.75) (width 0.2) (layer "B.Cu") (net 48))
 (segment (start 75.19 37.75) (end 68.23 30.79) (width 0.2) (layer "B.Cu") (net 48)))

